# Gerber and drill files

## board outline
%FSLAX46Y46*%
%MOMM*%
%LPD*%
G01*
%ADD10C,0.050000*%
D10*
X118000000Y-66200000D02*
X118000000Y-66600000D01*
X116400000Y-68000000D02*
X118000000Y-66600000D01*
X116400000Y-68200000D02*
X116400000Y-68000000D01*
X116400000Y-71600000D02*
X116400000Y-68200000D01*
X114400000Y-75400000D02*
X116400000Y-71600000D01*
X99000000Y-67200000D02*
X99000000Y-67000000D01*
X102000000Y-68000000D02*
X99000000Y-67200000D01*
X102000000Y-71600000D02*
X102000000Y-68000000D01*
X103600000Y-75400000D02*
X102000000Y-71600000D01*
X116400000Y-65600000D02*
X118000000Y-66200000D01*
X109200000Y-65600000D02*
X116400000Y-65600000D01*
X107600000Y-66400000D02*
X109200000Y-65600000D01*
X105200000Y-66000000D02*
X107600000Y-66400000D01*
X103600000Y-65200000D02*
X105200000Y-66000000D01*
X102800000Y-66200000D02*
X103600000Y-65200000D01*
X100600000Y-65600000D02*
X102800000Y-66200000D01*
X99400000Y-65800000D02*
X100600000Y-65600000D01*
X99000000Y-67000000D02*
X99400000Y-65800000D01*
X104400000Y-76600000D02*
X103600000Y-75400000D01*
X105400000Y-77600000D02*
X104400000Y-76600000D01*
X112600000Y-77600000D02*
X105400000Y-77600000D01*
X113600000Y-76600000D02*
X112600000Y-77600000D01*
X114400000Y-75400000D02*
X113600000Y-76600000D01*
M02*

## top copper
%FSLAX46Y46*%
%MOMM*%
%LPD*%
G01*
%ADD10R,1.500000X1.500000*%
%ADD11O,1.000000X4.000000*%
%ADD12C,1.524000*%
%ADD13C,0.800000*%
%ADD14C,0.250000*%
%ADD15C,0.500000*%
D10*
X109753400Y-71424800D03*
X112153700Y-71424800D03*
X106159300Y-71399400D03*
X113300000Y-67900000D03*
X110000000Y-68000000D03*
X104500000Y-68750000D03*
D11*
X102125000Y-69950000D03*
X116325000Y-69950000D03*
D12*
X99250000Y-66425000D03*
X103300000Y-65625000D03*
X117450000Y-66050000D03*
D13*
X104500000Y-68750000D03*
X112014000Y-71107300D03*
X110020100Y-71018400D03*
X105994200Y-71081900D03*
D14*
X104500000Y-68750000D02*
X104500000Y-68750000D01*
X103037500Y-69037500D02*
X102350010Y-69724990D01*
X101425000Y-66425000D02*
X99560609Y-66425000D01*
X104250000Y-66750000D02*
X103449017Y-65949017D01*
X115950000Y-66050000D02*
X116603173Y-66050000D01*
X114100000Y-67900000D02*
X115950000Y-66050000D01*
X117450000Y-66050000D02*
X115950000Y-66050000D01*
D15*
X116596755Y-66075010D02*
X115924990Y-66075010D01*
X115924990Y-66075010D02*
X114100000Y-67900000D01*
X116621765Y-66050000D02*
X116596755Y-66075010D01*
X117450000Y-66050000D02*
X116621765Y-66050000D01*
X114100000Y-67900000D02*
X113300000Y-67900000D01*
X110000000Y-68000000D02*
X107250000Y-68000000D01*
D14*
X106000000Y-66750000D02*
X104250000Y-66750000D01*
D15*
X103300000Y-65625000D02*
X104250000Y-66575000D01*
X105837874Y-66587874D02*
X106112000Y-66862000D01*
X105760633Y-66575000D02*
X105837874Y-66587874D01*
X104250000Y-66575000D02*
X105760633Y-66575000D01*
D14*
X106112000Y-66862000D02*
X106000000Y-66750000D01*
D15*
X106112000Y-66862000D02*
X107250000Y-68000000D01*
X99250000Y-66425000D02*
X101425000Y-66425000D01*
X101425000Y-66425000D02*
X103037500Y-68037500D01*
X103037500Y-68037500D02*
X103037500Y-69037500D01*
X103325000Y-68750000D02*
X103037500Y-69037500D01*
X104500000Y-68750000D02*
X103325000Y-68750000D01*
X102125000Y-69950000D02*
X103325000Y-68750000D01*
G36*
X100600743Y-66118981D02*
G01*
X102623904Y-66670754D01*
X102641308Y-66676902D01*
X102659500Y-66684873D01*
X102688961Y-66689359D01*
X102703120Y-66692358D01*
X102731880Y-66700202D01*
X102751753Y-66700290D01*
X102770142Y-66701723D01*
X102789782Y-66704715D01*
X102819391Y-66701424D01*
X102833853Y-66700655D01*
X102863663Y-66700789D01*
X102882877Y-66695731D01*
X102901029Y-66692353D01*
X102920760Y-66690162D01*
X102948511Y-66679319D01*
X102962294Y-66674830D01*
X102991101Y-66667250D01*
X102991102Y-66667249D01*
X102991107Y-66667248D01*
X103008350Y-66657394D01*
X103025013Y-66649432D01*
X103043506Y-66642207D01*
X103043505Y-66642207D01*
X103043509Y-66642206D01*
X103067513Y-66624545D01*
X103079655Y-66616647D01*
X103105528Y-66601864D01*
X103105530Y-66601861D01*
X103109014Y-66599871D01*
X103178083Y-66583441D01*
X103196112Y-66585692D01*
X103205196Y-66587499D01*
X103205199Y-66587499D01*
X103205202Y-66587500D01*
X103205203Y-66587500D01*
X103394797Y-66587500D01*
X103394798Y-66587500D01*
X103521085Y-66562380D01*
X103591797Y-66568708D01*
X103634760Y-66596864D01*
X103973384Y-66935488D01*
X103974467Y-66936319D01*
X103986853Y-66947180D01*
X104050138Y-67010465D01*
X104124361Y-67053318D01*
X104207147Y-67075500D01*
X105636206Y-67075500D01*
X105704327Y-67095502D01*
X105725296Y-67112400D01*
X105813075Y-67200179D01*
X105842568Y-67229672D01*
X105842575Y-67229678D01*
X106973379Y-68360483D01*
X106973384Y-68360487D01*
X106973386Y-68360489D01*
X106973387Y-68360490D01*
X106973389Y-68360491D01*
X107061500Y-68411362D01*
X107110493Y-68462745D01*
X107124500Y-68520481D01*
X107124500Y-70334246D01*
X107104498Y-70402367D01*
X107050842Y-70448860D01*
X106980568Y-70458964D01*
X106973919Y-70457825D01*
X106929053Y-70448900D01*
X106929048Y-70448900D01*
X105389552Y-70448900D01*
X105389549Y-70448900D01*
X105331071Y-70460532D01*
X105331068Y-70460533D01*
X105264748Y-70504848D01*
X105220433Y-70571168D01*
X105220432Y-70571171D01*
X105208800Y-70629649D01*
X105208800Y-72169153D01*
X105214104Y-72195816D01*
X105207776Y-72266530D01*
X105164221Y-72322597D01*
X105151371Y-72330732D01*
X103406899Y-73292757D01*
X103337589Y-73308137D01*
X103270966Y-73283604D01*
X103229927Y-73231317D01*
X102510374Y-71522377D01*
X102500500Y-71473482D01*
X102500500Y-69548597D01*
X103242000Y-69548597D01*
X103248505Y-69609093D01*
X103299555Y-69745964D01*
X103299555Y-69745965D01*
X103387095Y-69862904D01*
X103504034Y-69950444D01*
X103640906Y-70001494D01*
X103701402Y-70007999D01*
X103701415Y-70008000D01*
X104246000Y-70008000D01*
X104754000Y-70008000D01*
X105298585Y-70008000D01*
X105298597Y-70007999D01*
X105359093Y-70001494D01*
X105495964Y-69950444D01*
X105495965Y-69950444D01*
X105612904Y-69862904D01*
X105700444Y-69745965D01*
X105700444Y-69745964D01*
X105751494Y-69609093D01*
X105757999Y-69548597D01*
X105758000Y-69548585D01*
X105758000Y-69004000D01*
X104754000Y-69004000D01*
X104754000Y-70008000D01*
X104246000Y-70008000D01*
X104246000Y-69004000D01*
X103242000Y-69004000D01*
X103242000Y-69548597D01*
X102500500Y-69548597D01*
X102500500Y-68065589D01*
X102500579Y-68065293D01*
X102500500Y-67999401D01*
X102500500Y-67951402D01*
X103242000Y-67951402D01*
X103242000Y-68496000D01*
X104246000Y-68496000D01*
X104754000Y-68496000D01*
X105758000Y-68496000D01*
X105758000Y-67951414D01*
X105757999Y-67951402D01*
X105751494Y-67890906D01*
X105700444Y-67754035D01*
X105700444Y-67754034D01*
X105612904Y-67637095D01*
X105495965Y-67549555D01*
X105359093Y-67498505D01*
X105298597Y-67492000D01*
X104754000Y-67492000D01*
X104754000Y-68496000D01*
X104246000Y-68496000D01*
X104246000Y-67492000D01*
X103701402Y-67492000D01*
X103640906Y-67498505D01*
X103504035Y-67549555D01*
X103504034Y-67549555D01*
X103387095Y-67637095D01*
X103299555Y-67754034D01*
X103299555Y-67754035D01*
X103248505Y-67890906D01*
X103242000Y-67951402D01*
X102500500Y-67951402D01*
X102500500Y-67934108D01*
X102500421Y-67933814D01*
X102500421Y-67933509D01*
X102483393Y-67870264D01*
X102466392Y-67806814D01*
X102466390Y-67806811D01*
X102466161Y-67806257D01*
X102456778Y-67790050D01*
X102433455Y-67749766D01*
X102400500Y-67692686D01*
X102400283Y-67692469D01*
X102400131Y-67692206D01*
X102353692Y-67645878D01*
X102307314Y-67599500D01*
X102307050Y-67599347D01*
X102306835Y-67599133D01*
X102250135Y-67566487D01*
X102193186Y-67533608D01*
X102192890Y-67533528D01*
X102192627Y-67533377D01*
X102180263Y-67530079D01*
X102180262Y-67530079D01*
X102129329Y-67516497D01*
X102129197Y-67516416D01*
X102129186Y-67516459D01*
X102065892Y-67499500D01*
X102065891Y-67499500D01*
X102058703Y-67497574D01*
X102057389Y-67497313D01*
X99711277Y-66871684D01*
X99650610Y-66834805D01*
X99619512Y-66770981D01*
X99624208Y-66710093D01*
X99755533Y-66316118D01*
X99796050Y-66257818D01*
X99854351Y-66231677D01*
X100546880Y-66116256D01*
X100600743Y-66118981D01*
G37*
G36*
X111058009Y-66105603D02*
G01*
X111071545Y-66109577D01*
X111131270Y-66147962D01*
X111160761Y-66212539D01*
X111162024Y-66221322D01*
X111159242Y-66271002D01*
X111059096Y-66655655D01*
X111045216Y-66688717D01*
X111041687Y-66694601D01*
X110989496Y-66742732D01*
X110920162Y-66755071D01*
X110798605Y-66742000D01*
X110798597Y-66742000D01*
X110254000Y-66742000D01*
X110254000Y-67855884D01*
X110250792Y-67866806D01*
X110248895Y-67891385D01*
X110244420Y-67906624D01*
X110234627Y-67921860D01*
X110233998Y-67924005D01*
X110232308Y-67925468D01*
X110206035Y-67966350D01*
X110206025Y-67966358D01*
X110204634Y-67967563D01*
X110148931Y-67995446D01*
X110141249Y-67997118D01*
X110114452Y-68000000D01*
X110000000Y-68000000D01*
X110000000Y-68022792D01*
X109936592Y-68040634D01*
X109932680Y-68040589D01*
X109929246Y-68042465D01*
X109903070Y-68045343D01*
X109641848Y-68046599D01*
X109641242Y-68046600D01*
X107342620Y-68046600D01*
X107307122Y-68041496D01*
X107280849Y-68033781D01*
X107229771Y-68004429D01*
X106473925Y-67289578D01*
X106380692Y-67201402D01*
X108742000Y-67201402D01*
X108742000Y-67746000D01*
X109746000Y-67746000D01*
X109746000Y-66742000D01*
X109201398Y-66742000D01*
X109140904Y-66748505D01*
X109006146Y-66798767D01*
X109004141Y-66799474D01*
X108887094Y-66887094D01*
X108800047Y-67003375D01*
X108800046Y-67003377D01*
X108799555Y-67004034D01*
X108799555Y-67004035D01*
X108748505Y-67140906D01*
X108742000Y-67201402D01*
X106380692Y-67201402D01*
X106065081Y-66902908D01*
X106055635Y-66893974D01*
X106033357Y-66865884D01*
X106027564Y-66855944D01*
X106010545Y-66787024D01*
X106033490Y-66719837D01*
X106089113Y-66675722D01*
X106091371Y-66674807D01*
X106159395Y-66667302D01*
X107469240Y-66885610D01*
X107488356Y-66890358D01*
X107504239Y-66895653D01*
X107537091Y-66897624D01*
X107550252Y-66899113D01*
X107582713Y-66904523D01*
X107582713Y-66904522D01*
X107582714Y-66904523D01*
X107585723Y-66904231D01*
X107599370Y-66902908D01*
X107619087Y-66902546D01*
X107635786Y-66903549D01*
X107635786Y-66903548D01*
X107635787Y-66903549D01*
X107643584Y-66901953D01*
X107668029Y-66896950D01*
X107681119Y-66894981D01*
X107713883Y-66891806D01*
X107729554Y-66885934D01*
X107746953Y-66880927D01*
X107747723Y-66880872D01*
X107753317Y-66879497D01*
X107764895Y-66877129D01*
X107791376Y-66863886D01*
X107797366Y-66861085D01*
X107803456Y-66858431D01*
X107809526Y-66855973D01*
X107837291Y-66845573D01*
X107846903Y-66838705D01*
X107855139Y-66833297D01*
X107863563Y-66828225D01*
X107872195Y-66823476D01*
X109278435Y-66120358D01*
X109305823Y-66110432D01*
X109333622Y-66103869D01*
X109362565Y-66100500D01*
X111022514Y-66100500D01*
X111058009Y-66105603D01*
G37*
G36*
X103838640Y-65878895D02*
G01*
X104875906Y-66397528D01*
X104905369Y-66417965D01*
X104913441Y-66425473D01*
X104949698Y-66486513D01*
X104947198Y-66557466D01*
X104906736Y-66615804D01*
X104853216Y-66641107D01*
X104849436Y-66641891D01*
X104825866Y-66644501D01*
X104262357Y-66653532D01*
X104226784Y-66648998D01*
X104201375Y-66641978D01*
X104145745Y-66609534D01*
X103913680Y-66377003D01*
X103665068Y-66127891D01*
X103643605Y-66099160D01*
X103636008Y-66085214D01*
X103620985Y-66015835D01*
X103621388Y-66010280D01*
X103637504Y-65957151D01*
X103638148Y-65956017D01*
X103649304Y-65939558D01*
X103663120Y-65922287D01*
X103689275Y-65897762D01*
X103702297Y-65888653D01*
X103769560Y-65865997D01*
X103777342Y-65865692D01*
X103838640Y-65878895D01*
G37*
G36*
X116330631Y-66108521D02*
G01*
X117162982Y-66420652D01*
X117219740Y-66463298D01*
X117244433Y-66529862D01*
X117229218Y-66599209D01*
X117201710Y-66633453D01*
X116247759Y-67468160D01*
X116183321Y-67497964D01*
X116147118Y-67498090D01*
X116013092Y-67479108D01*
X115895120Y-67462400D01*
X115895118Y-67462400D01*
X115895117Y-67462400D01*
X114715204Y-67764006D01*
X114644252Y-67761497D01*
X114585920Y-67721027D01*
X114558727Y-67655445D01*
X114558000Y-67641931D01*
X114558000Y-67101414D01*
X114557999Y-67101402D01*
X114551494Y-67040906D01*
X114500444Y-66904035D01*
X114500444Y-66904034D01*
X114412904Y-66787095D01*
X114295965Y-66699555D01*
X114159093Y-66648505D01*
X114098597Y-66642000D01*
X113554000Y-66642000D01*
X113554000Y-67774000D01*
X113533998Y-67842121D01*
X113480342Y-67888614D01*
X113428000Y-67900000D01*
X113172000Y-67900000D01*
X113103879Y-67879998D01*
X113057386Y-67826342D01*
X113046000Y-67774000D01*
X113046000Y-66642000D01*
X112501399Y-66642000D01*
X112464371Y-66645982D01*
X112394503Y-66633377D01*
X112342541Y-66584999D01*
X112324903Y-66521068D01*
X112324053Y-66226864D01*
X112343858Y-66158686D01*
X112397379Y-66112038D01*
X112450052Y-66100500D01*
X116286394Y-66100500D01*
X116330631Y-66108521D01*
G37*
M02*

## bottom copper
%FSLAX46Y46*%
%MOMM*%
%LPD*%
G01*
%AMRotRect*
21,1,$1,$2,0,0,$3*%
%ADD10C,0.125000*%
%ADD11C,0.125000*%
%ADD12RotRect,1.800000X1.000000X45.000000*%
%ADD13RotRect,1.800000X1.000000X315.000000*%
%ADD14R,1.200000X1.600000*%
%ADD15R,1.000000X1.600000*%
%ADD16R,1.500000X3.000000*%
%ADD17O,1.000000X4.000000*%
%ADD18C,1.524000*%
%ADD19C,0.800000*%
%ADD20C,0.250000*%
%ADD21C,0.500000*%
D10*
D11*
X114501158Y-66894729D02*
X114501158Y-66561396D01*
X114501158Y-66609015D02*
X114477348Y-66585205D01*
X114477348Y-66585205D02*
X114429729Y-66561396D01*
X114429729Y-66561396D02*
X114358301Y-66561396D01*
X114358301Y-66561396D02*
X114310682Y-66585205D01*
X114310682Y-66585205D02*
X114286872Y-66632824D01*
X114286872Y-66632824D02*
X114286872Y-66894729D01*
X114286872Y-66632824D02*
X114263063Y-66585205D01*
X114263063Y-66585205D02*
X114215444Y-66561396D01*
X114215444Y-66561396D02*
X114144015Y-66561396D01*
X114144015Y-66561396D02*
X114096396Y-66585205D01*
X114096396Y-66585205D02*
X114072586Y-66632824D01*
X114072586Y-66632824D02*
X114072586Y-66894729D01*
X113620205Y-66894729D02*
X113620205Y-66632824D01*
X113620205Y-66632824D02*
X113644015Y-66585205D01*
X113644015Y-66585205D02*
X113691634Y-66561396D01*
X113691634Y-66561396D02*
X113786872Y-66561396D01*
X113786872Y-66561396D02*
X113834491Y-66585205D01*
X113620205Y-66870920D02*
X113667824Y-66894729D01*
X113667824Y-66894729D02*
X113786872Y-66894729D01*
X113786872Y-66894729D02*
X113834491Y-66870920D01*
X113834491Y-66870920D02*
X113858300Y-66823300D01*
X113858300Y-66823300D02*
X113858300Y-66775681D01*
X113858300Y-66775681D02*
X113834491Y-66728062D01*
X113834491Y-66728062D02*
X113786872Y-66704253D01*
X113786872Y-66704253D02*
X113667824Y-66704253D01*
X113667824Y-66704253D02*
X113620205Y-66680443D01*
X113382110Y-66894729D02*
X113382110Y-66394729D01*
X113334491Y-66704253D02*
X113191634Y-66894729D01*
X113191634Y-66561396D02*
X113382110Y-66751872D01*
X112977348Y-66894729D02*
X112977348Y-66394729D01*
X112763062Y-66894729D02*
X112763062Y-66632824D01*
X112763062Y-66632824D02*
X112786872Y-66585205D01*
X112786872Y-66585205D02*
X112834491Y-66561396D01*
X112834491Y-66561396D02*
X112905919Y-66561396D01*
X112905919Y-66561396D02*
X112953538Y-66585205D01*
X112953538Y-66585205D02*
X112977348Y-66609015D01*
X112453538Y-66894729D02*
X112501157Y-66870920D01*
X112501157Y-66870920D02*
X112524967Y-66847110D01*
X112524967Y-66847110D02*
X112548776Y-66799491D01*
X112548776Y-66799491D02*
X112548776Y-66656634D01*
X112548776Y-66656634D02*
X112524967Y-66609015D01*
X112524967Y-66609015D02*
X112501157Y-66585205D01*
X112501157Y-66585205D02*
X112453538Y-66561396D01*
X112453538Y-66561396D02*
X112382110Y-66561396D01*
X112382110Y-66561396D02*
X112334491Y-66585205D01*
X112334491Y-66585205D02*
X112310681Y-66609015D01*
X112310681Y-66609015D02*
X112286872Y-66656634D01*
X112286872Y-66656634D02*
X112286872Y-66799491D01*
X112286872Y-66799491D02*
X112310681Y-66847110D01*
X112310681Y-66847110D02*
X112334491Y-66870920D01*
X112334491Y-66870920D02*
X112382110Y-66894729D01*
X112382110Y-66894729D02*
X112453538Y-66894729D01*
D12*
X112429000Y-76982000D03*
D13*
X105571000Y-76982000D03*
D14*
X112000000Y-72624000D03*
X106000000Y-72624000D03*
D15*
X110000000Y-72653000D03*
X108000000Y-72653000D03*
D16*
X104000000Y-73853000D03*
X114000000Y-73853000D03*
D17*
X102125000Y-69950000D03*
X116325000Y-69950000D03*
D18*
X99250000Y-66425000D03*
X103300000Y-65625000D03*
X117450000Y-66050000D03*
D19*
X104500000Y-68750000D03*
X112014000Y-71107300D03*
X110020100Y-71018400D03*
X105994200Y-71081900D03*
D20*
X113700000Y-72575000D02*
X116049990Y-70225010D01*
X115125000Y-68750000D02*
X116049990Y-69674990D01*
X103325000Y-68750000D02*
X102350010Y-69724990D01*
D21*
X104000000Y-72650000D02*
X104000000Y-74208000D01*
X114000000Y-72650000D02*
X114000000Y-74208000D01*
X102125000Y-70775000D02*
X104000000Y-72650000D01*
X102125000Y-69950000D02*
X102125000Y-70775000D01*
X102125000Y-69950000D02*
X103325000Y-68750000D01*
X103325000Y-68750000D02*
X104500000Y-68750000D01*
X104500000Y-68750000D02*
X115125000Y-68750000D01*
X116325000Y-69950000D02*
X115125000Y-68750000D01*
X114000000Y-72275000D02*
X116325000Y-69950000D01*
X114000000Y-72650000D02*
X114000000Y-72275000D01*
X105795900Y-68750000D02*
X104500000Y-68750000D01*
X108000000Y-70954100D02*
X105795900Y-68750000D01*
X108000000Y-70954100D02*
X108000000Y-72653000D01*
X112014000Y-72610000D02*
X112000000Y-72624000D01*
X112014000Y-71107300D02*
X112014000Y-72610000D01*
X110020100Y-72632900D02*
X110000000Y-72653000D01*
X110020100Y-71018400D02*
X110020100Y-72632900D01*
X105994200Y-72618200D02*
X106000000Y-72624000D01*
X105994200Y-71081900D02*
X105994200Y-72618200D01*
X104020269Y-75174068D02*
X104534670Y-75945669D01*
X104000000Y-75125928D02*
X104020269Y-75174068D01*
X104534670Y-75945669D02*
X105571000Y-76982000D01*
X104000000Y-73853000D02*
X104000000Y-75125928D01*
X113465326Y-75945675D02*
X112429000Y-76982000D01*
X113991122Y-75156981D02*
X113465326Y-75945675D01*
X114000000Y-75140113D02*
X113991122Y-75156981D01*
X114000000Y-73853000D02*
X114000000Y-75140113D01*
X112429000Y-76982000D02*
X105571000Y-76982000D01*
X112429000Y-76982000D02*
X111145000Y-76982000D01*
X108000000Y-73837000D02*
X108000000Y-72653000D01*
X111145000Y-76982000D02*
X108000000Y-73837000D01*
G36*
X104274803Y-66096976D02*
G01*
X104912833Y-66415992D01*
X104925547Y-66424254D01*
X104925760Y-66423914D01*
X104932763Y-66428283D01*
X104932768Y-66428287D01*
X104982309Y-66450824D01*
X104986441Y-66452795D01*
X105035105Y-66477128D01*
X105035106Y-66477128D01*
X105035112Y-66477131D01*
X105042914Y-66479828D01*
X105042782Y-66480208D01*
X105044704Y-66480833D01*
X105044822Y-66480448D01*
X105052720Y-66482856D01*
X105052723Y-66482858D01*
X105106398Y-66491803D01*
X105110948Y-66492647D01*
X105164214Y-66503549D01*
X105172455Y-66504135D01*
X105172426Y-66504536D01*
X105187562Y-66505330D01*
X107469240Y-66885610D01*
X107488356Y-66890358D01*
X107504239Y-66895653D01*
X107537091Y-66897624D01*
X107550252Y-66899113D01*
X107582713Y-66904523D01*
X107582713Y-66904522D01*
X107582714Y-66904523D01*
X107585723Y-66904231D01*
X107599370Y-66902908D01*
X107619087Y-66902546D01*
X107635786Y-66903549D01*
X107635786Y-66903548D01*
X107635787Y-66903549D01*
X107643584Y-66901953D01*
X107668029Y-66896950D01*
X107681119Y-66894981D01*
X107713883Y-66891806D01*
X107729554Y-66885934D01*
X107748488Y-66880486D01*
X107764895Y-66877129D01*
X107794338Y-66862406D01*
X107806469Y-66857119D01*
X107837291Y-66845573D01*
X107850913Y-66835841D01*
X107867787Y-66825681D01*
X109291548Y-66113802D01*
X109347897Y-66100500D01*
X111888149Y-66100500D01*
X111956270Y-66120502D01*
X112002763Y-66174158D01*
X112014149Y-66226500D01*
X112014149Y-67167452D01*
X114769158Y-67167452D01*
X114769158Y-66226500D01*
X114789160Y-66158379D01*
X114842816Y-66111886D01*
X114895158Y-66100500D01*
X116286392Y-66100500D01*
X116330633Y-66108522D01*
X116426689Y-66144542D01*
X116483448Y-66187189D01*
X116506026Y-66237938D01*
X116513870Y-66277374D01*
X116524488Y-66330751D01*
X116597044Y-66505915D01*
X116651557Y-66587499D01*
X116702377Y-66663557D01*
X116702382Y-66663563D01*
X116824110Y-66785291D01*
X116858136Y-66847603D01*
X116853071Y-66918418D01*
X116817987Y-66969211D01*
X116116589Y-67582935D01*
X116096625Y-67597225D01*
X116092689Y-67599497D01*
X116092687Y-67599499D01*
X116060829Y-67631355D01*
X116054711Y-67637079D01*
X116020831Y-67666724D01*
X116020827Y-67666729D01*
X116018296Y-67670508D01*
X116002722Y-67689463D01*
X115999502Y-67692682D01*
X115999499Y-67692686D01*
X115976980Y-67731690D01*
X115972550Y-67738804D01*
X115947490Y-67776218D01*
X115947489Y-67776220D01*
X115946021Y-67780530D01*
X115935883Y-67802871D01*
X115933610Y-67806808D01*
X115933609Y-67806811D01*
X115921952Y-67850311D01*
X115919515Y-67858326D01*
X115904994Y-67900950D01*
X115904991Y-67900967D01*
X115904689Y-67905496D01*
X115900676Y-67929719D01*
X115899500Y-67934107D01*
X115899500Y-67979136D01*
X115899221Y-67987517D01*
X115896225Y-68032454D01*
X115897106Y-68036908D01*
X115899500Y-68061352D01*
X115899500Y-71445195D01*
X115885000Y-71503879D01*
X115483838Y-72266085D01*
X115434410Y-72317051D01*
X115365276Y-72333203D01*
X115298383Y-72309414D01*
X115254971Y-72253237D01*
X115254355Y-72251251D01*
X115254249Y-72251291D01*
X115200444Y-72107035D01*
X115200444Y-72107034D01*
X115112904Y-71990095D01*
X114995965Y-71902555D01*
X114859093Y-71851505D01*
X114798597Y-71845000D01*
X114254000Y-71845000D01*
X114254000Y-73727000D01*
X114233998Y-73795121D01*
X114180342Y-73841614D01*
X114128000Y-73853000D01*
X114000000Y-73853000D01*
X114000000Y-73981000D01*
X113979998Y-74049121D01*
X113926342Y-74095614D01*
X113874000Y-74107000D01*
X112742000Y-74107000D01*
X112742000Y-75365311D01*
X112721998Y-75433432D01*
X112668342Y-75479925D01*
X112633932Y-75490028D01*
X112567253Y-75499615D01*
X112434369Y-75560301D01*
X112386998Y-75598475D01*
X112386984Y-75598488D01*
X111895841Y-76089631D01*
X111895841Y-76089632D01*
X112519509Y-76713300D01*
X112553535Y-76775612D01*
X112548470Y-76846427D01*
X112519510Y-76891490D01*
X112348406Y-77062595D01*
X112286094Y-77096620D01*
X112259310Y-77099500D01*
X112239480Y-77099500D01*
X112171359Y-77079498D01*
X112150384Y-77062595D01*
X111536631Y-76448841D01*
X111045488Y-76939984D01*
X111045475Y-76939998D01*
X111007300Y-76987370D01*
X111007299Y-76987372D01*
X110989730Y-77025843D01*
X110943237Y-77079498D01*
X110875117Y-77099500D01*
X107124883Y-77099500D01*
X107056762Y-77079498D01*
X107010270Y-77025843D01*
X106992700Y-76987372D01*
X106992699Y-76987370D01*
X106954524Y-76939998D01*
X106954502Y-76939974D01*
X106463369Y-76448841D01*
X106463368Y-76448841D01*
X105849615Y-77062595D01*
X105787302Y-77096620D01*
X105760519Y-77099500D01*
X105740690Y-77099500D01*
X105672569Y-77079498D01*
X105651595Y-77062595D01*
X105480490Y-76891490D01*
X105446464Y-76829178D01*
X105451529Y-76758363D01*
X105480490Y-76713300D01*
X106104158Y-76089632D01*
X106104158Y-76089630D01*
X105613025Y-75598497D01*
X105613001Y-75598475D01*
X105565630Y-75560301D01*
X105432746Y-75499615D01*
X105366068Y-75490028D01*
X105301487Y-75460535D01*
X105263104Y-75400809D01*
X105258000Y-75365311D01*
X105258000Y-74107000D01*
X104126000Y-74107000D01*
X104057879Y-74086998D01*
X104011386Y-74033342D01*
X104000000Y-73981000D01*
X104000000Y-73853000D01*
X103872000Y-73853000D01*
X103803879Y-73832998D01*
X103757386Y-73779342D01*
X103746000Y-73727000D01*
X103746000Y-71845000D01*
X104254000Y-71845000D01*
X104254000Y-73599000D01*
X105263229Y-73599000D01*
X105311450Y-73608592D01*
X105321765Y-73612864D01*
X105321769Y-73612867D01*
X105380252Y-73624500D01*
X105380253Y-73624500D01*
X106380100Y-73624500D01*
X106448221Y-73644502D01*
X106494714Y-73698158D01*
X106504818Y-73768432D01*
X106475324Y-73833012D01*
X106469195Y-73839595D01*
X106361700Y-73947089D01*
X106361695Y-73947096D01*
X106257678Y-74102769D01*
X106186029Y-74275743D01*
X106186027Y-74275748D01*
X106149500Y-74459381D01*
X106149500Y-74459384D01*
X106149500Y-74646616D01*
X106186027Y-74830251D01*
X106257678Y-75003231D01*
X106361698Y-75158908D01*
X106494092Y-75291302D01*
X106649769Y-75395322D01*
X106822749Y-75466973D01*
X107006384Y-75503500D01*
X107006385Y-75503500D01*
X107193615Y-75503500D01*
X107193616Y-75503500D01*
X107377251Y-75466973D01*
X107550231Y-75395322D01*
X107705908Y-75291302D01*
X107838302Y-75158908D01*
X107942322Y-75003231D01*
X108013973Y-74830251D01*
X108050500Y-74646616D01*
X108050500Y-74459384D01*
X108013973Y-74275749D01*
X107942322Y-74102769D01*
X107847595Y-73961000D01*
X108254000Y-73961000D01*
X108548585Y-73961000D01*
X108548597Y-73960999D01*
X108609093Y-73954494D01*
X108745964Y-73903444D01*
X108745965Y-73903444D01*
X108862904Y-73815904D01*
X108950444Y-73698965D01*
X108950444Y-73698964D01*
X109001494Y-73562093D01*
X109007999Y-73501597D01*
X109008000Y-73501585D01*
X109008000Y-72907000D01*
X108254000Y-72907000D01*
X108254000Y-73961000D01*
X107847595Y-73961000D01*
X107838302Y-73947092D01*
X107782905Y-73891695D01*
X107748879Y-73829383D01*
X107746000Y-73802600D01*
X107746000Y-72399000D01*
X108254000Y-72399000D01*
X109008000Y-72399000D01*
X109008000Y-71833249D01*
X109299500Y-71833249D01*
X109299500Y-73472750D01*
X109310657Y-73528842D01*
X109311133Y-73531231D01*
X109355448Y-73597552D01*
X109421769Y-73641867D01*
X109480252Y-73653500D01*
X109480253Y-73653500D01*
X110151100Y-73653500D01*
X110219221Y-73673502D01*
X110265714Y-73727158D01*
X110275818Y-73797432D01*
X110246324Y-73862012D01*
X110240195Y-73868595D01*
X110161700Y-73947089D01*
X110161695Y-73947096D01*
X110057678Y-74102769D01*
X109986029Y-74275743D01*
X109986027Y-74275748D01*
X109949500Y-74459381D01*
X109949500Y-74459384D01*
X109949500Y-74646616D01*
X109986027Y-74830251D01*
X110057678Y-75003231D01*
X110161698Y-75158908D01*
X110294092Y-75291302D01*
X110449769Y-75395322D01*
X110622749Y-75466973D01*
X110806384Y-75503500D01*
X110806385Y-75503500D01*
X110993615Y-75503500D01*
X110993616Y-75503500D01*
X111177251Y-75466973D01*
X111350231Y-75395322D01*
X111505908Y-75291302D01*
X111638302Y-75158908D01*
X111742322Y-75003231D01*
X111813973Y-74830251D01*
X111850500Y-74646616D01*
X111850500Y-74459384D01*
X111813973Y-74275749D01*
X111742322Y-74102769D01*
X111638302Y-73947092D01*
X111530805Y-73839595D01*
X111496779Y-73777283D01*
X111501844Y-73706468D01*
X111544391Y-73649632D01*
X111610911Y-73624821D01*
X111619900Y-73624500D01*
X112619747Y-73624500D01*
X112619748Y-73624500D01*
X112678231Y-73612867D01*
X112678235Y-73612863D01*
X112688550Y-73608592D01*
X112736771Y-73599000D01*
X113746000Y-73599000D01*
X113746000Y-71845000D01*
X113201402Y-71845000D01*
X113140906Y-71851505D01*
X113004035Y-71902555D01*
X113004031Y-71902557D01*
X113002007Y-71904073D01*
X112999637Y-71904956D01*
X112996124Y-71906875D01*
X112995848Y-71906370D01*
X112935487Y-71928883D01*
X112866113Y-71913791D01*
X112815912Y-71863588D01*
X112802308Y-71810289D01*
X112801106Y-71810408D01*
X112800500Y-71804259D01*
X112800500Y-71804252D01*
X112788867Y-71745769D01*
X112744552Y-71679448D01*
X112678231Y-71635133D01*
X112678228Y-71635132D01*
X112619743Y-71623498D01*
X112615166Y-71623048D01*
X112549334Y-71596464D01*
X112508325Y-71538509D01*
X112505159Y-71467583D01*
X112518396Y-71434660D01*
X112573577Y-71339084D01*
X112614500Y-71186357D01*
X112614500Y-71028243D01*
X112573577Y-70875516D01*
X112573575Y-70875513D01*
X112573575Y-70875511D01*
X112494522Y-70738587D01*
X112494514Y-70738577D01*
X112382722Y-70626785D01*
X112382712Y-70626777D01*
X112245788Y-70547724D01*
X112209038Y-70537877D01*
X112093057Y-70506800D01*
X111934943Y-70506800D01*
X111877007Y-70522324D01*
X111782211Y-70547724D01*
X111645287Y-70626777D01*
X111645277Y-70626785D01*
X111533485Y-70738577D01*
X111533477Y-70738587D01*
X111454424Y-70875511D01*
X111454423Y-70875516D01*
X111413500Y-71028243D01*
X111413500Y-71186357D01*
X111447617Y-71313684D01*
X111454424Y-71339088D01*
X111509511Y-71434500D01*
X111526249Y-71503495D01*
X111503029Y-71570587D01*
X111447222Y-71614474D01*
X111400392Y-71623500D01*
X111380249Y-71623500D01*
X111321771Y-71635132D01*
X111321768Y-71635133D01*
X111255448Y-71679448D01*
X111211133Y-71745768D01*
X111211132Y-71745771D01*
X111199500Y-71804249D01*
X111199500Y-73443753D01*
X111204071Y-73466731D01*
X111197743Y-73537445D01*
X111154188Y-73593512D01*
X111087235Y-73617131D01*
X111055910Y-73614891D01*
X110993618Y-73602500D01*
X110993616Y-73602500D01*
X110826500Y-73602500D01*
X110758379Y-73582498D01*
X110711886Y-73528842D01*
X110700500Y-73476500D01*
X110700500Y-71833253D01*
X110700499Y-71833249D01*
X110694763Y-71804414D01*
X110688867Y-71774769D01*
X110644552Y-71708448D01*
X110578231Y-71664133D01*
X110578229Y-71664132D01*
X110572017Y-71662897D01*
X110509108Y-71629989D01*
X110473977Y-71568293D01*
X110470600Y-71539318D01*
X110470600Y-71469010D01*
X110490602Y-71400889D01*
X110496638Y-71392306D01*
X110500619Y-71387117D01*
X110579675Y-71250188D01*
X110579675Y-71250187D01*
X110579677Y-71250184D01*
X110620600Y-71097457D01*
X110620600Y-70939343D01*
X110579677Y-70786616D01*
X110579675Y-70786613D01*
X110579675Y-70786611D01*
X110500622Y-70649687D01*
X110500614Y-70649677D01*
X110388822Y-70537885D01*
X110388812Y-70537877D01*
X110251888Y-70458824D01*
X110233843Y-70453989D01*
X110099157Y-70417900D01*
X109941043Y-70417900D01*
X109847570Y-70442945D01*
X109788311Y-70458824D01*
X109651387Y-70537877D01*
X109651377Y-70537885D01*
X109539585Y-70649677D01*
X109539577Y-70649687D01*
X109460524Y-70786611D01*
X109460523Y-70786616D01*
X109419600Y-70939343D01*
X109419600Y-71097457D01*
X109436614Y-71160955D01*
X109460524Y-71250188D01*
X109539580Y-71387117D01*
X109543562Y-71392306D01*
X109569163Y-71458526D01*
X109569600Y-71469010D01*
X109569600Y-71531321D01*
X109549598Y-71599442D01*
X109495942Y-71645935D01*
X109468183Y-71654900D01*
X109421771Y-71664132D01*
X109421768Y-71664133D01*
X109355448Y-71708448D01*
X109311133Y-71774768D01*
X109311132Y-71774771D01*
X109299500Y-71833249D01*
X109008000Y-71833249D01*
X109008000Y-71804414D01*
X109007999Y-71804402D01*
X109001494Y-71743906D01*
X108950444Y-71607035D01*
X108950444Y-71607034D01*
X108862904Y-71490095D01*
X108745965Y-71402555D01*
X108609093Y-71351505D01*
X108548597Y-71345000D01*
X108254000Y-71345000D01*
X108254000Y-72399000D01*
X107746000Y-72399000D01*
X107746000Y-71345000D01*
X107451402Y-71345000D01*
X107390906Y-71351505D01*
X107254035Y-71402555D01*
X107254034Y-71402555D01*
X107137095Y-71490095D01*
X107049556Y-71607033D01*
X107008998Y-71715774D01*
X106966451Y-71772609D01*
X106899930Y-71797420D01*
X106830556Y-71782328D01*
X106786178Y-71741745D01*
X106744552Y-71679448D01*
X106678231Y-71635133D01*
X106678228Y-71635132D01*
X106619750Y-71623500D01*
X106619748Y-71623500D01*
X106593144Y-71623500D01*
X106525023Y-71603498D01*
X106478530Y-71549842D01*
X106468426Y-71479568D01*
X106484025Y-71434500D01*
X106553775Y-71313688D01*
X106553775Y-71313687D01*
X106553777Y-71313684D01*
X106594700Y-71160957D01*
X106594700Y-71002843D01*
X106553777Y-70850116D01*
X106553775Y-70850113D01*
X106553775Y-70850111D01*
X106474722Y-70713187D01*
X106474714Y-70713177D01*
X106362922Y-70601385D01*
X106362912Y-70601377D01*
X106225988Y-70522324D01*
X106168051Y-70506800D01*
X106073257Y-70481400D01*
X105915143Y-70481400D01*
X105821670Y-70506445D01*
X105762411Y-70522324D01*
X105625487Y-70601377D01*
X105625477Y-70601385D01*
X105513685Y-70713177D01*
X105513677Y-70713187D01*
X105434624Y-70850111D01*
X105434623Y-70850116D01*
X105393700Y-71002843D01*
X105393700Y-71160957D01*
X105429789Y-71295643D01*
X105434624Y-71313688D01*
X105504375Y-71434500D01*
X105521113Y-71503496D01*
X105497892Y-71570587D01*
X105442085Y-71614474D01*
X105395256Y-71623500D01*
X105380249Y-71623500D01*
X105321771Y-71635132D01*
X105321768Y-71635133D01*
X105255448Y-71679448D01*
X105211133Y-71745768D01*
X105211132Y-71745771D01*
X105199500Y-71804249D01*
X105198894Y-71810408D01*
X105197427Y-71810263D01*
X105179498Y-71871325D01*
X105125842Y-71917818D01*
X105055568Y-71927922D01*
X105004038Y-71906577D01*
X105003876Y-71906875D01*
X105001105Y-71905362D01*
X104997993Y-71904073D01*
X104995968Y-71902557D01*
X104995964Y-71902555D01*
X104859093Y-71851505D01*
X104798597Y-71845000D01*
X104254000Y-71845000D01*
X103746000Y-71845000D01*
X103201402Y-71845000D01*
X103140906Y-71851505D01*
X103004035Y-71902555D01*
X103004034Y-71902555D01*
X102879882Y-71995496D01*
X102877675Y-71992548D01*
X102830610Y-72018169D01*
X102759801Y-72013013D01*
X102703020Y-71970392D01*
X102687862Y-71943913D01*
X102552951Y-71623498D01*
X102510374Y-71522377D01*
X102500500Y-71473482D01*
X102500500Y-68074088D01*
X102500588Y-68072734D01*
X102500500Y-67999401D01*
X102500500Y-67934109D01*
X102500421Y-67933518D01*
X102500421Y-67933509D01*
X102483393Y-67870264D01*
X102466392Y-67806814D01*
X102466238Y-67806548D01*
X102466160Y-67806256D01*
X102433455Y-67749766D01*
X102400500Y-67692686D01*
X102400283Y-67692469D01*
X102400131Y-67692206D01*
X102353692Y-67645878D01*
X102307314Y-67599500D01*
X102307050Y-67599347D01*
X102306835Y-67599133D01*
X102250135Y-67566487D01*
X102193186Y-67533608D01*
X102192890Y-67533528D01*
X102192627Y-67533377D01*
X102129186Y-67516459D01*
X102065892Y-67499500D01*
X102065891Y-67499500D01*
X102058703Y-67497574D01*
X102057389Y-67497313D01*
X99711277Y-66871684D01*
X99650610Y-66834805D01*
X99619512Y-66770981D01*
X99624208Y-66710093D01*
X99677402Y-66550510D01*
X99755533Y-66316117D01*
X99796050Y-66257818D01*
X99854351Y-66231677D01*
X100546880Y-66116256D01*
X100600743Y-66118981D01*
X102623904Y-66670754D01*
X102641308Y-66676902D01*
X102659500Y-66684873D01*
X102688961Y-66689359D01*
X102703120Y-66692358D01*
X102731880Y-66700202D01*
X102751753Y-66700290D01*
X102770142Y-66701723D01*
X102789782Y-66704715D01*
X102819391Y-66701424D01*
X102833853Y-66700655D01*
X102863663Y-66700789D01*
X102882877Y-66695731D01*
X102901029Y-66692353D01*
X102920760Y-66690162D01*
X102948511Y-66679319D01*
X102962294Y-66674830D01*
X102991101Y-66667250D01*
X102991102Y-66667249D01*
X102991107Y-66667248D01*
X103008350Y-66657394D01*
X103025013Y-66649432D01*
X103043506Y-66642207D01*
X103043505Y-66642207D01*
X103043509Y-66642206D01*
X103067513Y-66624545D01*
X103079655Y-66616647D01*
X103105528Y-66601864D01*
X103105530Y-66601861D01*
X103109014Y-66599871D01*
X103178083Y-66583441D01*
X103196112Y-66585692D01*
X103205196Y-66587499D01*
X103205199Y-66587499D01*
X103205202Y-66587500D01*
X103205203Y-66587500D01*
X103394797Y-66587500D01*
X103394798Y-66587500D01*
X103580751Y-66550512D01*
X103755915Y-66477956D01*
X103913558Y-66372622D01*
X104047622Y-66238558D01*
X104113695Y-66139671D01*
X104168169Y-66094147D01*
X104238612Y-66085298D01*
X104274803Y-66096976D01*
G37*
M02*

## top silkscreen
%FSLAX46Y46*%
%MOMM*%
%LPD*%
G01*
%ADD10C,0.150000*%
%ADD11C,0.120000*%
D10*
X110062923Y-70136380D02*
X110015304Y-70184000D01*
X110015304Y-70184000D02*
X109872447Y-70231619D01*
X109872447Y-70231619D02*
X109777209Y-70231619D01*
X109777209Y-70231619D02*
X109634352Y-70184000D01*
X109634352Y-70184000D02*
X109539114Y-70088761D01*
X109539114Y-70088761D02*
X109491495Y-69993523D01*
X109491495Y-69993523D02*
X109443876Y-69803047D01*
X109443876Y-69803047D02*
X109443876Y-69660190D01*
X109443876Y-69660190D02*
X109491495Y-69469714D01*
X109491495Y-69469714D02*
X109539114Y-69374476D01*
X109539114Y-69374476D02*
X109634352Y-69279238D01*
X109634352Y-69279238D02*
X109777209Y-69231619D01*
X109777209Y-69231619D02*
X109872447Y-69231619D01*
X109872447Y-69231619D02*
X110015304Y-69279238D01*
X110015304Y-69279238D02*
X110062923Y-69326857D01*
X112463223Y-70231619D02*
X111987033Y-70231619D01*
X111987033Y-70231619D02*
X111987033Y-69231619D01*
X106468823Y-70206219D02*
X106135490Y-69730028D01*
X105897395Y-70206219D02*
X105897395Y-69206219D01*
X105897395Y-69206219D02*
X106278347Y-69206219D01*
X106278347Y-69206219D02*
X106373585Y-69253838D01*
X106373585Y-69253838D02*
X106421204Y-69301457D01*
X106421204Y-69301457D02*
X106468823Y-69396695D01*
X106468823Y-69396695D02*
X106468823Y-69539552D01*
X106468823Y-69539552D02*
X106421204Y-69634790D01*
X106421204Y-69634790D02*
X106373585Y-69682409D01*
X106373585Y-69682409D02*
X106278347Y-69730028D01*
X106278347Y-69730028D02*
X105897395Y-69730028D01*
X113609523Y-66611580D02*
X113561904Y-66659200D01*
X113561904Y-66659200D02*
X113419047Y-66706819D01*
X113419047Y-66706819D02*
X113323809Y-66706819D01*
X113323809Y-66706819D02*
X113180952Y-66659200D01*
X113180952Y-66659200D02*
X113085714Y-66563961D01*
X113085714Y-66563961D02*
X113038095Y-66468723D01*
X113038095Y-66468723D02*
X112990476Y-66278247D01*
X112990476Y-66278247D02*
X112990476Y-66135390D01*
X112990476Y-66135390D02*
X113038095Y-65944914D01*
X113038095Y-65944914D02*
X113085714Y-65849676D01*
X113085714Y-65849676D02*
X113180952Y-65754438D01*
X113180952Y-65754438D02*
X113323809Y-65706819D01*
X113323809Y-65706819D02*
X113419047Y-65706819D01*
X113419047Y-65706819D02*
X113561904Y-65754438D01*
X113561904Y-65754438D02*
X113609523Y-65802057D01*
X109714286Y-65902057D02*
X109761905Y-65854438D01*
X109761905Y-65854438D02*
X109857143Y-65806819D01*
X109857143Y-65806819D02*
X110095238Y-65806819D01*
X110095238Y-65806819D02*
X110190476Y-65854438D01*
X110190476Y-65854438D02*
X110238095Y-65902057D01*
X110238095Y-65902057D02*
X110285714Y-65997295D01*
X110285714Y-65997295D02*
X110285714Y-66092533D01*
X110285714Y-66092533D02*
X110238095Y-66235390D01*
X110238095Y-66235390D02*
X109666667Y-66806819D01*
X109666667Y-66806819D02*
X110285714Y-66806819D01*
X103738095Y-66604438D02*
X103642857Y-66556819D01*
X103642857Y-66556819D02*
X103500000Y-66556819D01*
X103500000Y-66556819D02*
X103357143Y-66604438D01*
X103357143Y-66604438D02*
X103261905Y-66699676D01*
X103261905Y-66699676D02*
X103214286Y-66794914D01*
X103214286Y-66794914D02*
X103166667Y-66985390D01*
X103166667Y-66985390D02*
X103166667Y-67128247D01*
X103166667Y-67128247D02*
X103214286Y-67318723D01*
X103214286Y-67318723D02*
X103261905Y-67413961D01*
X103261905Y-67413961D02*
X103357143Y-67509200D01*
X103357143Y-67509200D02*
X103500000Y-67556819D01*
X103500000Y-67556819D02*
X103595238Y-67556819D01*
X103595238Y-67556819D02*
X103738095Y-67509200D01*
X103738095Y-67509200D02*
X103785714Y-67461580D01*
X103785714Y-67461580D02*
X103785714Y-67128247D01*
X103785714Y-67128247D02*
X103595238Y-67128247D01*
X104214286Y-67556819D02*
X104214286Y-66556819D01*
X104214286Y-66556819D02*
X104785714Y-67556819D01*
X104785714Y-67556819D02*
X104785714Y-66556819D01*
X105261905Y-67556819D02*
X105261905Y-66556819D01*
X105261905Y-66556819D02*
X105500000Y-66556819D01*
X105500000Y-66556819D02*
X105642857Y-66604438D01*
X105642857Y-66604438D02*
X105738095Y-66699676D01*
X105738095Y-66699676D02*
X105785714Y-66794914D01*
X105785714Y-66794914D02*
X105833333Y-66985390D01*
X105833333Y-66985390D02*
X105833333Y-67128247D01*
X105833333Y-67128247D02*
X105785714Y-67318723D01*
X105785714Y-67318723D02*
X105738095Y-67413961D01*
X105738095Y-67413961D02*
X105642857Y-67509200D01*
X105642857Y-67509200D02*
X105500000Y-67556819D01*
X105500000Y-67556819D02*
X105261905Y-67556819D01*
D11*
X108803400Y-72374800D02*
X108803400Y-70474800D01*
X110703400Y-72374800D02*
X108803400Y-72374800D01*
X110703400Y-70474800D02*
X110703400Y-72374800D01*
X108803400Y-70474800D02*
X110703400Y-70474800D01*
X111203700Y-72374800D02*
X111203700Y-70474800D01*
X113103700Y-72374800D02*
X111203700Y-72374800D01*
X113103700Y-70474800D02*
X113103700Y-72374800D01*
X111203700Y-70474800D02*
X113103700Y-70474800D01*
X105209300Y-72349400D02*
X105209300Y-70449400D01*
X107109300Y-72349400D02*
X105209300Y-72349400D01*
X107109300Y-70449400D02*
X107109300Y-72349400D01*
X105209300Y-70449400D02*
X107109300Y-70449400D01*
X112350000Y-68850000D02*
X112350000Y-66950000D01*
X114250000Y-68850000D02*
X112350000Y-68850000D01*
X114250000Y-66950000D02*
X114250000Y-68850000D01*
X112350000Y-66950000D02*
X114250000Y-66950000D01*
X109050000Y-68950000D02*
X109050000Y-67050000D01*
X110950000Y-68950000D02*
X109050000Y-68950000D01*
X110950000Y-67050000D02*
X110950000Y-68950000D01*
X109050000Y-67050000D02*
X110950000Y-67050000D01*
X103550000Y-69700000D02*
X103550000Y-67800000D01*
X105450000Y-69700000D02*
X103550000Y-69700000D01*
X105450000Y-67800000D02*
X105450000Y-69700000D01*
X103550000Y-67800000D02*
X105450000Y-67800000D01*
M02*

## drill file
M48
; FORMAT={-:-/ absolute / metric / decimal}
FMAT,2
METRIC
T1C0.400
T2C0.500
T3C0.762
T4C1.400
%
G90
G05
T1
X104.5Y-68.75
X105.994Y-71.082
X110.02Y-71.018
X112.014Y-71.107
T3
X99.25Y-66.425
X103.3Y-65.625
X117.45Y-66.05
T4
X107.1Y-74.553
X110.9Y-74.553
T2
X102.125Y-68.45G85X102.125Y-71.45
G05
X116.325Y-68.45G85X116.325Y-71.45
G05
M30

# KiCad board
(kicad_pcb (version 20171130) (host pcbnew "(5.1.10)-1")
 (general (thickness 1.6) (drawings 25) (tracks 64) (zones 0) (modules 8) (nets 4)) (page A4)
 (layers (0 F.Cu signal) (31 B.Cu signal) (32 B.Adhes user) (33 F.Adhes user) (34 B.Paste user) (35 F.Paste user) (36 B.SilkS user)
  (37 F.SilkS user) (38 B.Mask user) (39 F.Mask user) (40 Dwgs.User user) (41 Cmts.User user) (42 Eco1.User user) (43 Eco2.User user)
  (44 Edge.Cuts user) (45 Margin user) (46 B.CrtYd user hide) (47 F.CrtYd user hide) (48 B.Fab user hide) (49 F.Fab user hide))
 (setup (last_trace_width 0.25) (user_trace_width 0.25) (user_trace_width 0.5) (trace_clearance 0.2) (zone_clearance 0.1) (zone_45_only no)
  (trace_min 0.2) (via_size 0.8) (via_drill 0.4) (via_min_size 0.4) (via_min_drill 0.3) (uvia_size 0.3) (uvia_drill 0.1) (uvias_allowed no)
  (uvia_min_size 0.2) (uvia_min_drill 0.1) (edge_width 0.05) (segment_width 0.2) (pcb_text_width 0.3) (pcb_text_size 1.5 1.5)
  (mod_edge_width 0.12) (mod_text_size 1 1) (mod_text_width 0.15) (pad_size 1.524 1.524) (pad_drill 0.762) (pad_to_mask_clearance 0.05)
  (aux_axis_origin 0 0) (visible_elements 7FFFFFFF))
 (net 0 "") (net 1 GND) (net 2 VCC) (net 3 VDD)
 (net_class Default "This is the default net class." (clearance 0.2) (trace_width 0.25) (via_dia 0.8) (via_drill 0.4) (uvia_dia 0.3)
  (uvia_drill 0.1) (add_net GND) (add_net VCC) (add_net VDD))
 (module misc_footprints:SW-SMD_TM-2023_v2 (layer B.Cu) (at 109 74.803)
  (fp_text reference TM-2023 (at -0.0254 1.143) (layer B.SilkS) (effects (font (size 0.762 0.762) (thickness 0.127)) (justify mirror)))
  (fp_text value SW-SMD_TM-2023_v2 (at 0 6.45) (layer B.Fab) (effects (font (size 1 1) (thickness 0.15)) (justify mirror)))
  (pad GND smd rect (at 3.429 2.179 45) (size 1.8 1) (layers B.Cu B.Paste B.Mask) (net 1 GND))
  (pad GND smd rect (at -3.429 2.179 315) (size 1.8 1) (layers B.Cu B.Paste B.Mask) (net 1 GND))
  (pad 1 smd rect (at 3 -2.179) (size 1.2 1.6) (layers B.Cu B.Paste B.Mask))
  (pad 2 smd rect (at -3 -2.179) (size 1.2 1.6) (layers B.Cu B.Paste B.Mask))
  (pad C smd rect (at 1 -2.15) (size 1 1.6) (layers B.Cu B.Paste B.Mask))
  (pad T smd rect (at -1 -2.15) (size 1 1.6) (layers B.Cu B.Paste B.Mask) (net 1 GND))
  (pad GND smd rect (at -5 -0.95) (size 1.5 3) (layers B.Cu B.Paste B.Mask) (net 1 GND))
  (pad 6 smd rect (at 5 -0.95) (size 1.5 3) (layers B.Cu B.Paste B.Mask) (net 1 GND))
  (pad "" np_thru_hole circle (at 1.9 -0.25) (size 1.4 1.4) (drill 1.4) (layers *.Cu *.Mask))
  (pad "" np_thru_hole circle (at -1.9 -0.25) (size 1.4 1.4) (drill 1.4) (layers *.Cu *.Mask)))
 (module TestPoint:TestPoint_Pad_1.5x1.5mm (layer F.Cu) (at 109.7534 71.4248)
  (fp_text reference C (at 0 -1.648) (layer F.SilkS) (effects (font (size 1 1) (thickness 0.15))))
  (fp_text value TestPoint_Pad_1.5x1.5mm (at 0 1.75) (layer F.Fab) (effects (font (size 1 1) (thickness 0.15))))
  (fp_line (start -0.95 0.95) (end -0.95 -0.95) (layer F.SilkS) (width 0.12))
  (fp_line (start 0.95 0.95) (end -0.95 0.95) (layer F.SilkS) (width 0.12))
  (fp_line (start 0.95 -0.95) (end 0.95 0.95) (layer F.SilkS) (width 0.12))
  (fp_line (start -0.95 -0.95) (end 0.95 -0.95) (layer F.SilkS) (width 0.12))
  (pad 1 smd rect (at 0 0) (size 1.5 1.5) (layers F.Cu F.Mask)))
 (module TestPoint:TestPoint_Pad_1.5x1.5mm (layer F.Cu) (at 112.1537 71.4248)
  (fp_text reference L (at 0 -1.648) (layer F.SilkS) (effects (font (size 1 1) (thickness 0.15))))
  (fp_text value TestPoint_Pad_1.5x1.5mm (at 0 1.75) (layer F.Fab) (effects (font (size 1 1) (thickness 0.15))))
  (fp_line (start -0.95 0.95) (end -0.95 -0.95) (layer F.SilkS) (width 0.12))
  (fp_line (start 0.95 0.95) (end -0.95 0.95) (layer F.SilkS) (width 0.12))
  (fp_line (start 0.95 -0.95) (end 0.95 0.95) (layer F.SilkS) (width 0.12))
  (fp_line (start -0.95 -0.95) (end 0.95 -0.95) (layer F.SilkS) (width 0.12))
  (pad 1 smd rect (at 0 0) (size 1.5 1.5) (layers F.Cu F.Mask)))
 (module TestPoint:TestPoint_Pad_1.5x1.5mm (layer F.Cu) (at 106.1593 71.3994)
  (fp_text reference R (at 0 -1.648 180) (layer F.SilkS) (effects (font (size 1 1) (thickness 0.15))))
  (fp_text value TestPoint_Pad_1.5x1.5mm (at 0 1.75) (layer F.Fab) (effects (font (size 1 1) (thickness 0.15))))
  (fp_line (start -0.95 0.95) (end -0.95 -0.95) (layer F.SilkS) (width 0.12))
  (fp_line (start 0.95 0.95) (end -0.95 0.95) (layer F.SilkS) (width 0.12))
  (fp_line (start 0.95 -0.95) (end 0.95 0.95) (layer F.SilkS) (width 0.12))
  (fp_line (start -0.95 -0.95) (end 0.95 -0.95) (layer F.SilkS) (width 0.12))
  (pad 1 smd rect (at 0 0) (size 1.5 1.5) (layers F.Cu F.Mask)))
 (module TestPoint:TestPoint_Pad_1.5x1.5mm (layer F.Cu) (at 113.3 67.9)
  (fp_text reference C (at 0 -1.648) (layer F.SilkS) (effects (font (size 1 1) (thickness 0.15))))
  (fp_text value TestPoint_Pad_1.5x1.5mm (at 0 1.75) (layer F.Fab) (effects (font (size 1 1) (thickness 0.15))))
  (fp_line (start -0.95 0.95) (end -0.95 -0.95) (layer F.SilkS) (width 0.12))
  (fp_line (start 0.95 0.95) (end -0.95 0.95) (layer F.SilkS) (width 0.12))
  (fp_line (start 0.95 -0.95) (end 0.95 0.95) (layer F.SilkS) (width 0.12))
  (fp_line (start -0.95 -0.95) (end 0.95 -0.95) (layer F.SilkS) (width 0.12))
  (pad 1 smd rect (at 0 0) (size 1.5 1.5) (layers F.Cu F.Mask) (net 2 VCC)))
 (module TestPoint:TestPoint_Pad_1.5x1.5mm (layer F.Cu) (at 110 68)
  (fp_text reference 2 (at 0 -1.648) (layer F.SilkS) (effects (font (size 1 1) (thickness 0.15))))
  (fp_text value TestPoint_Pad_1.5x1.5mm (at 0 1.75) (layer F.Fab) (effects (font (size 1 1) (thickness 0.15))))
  (fp_line (start -0.95 0.95) (end -0.95 -0.95) (layer F.SilkS) (width 0.12))
  (fp_line (start 0.95 0.95) (end -0.95 0.95) (layer F.SilkS) (width 0.12))
  (fp_line (start 0.95 -0.95) (end 0.95 0.95) (layer F.SilkS) (width 0.12))
  (fp_line (start -0.95 -0.95) (end 0.95 -0.95) (layer F.SilkS) (width 0.12))
  (pad 1 smd rect (at 0 0) (size 1.5 1.5) (layers F.Cu F.Mask) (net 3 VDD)))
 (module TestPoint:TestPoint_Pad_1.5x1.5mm (layer F.Cu) (at 104.5 68.75)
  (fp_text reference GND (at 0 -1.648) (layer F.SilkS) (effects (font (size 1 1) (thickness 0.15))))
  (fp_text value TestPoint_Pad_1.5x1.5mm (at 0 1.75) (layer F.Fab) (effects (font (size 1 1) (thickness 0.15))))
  (fp_line (start -0.95 0.95) (end -0.95 -0.95) (layer F.SilkS) (width 0.12))
  (fp_line (start 0.95 0.95) (end -0.95 0.95) (layer F.SilkS) (width 0.12))
  (fp_line (start 0.95 -0.95) (end 0.95 0.95) (layer F.SilkS) (width 0.12))
  (fp_line (start -0.95 -0.95) (end 0.95 -0.95) (layer F.SilkS) (width 0.12))
  (pad 1 smd rect (at 0 0) (size 1.5 1.5) (layers F.Cu F.Mask) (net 1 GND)))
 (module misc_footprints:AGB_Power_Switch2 (layer F.Cu) (at 108.4 70.2)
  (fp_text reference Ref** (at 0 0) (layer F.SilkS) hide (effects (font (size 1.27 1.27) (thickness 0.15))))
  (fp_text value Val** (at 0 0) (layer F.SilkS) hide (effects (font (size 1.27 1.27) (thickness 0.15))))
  (pad 3 thru_hole oval (at -6.275 -0.25) (size 1 4) (drill oval 0.5 3.5) (layers *.Cu *.Mask) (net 1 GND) (zone_connect 2))
  (pad 3 thru_hole oval (at 7.925 -0.25) (size 1 4) (drill oval 0.5 3.5) (layers *.Cu *.Mask) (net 1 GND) (zone_connect 2))
  (pad 3 thru_hole circle (at -9.15 -3.775) (size 1.524 1.524) (drill 0.762) (layers *.Cu *.Mask) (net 1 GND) (zone_connect 2))
  (pad 2 thru_hole circle (at -5.1 -4.575) (size 1.524 1.524) (drill 0.762) (layers *.Cu *.Mask) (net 3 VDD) (zone_connect 2))
  (pad 1 thru_hole circle (at 9.05 -4.15) (size 1.524 1.524) (drill 0.762) (layers *.Cu *.Mask) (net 2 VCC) (zone_connect 2)))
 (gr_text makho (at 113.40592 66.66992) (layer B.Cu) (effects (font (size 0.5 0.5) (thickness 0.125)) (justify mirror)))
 (gr_line (start 118 66.2) (end 118 66.6) (layer Edge.Cuts) (width 0.05))
 (gr_line (start 116.4 68) (end 118 66.6) (layer Edge.Cuts) (width 0.05))
 (gr_line (start 116.4 68.2) (end 116.4 68) (layer Edge.Cuts) (width 0.05))
 (gr_line (start 116.4 71.6) (end 116.4 68.2) (layer Edge.Cuts) (width 0.05))
 (gr_line (start 114.4 75.4) (end 116.4 71.6) (layer Edge.Cuts) (width 0.05))
 (gr_line (start 99 67.2) (end 99 67) (layer Edge.Cuts) (width 0.05))
 (gr_line (start 102 68) (end 99 67.2) (layer Edge.Cuts) (width 0.05))
 (gr_line (start 102 71.6) (end 102 68) (layer Edge.Cuts) (width 0.05))
 (gr_line (start 103.6 75.4) (end 102 71.6) (layer Edge.Cuts) (width 0.05))
 (gr_line (start 116.4 65.6) (end 118 66.2) (layer Edge.Cuts) (width 0.05))
 (gr_line (start 109.2 65.6) (end 116.4 65.6) (layer Edge.Cuts) (width 0.05))
 (gr_line (start 107.6 66.4) (end 109.2 65.6) (layer Edge.Cuts) (width 0.05))
 (gr_line (start 105.2 66) (end 107.6 66.4) (layer Edge.Cuts) (width 0.05))
 (gr_line (start 103.6 65.2) (end 105.2 66) (layer Edge.Cuts) (width 0.05))
 (gr_line (start 102.8 66.2) (end 103.6 65.2) (layer Edge.Cuts) (width 0.05))
 (gr_line (start 100.6 65.6) (end 102.8 66.2) (layer Edge.Cuts) (width 0.05))
 (gr_line (start 99.4 65.8) (end 100.6 65.6) (layer Edge.Cuts) (width 0.05))
 (gr_line (start 99 67) (end 99.4 65.8) (layer Edge.Cuts) (width 0.05))
 (gr_line (start 104.4 76.6) (end 103.6 75.4) (layer Edge.Cuts) (width 0.05))
 (gr_line (start 105.4 77.6) (end 104.4 76.6) (layer Edge.Cuts) (width 0.05))
 (gr_line (start 112.6 77.6) (end 105.4 77.6) (layer Edge.Cuts) (width 0.05))
 (gr_line (start 113.6 76.6) (end 112.6 77.6) (layer Edge.Cuts) (width 0.05))
 (gr_line (start 114.4 75.4) (end 113.6 76.6) (layer Edge.Cuts) (width 0.05))
 (segment (start 113.7 72.575) (end 116.04999 70.22501) (width 0.25) (layer B.Cu) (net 1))
 (segment (start 104.5 68.75) (end 104.5 68.75) (width 0.25) (layer F.Cu) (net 1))
 (segment (start 103.0375 69.0375) (end 102.35001 69.72499) (width 0.25) (layer F.Cu) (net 1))
 (segment (start 101.425 66.425) (end 99.560609 66.425) (width 0.25) (layer F.Cu) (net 1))
 (segment (start 104.25 66.75) (end 103.449017 65.949017) (width 0.25) (layer F.Cu) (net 3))
 (segment (start 115.95 66.05) (end 116.603173 66.05) (width 0.25) (layer F.Cu) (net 2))
 (segment (start 114.1 67.9) (end 115.95 66.05) (width 0.25) (layer F.Cu) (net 2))
 (segment (start 117.45 66.05) (end 115.95 66.05) (width 0.25) (layer F.Cu) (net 2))
 (via (at 104.5 68.75) (size 0.8) (drill 0.4) (layers F.Cu B.Cu) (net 1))
 (segment (start 115.125 68.75) (end 116.04999 69.67499) (width 0.25) (layer B.Cu) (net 1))
 (segment (start 103.325 68.75) (end 102.35001 69.72499) (width 0.25) (layer B.Cu) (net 1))
 (segment (start 104 72.65) (end 104 74.208) (width 0.5) (layer B.Cu) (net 1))
 (segment (start 114 72.65) (end 114 74.208) (width 0.5) (layer B.Cu) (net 1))
 (segment (start 116.596755 66.07501) (end 115.92499 66.07501) (width 0.5) (layer F.Cu) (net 2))
 (segment (start 115.92499 66.07501) (end 114.1 67.9) (width 0.5) (layer F.Cu) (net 2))
 (segment (start 116.621765 66.05) (end 116.596755 66.07501) (width 0.5) (layer F.Cu) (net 2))
 (segment (start 117.45 66.05) (end 116.621765 66.05) (width 0.5) (layer F.Cu) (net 2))
 (segment (start 114.1 67.9) (end 113.3 67.9) (width 0.5) (layer F.Cu) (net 2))
 (segment (start 110 68) (end 107.25 68) (width 0.5) (layer F.Cu) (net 3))
 (segment (start 106 66.75) (end 104.25 66.75) (width 0.25) (layer F.Cu) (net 3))
 (segment (start 103.3 65.625) (end 104.25 66.575) (width 0.5) (layer F.Cu) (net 3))
 (segment (start 105.837874 66.587874) (end 106.112 66.862) (width 0.5) (layer F.Cu) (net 3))
 (segment (start 105.760633 66.575) (end 105.837874 66.587874) (width 0.5) (layer F.Cu) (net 3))
 (segment (start 104.25 66.575) (end 105.760633 66.575) (width 0.5) (layer F.Cu) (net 3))
 (segment (start 106.112 66.862) (end 106 66.75) (width 0.25) (layer F.Cu) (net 3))
 (segment (start 106.112 66.862) (end 107.25 68) (width 0.5) (layer F.Cu) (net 3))
 (segment (start 99.25 66.425) (end 101.425 66.425) (width 0.5) (layer F.Cu) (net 1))
 (segment (start 101.425 66.425) (end 103.0375 68.0375) (width 0.5) (layer F.Cu) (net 1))
 (segment (start 103.0375 68.0375) (end 103.0375 69.0375) (width 0.5) (layer F.Cu) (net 1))
 (segment (start 103.325 68.75) (end 103.0375 69.0375) (width 0.5) (layer F.Cu) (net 1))
 (segment (start 104.5 68.75) (end 103.325 68.75) (width 0.5) (layer F.Cu) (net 1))
 (segment (start 102.125 69.95) (end 103.325 68.75) (width 0.5) (layer F.Cu) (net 1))
 (segment (start 102.125 70.775) (end 104 72.65) (width 0.5) (layer B.Cu) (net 1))
 (segment (start 102.125 69.95) (end 102.125 70.775) (width 0.5) (layer B.Cu) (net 1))
 (segment (start 102.125 69.95) (end 103.325 68.75) (width 0.5) (layer B.Cu) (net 1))
 (segment (start 103.325 68.75) (end 104.5 68.75) (width 0.5) (layer B.Cu) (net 1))
 (segment (start 104.5 68.75) (end 115.125 68.75) (width 0.5) (layer B.Cu) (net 1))
 (segment (start 116.325 69.95) (end 115.125 68.75) (width 0.5) (layer B.Cu) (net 1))
 (segment (start 114 72.275) (end 116.325 69.95) (width 0.5) (layer B.Cu) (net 1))
 (segment (start 114 72.65) (end 114 72.275) (width 0.5) (layer B.Cu) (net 1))
 (segment (start 105.7959 68.75) (end 104.5 68.75) (width 0.5) (layer B.Cu) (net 1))
 (segment (start 108 70.9541) (end 105.7959 68.75) (width 0.5) (layer B.Cu) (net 1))
 (via (at 112.014 71.1073) (size 0.8) (drill 0.4) (layers F.Cu B.Cu) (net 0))
 (via (at 110.0201 71.0184) (size 0.8) (drill 0.4) (layers F.Cu B.Cu) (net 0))
 (via (at 105.9942 71.0819) (size 0.8) (drill 0.4) (layers F.Cu B.Cu) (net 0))
 (segment (start 108 70.9541) (end 108 72.653) (width 0.5) (layer B.Cu) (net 1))
 (segment (start 112.014 72.61) (end 112 72.624) (width 0.5) (layer B.Cu) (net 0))
 (segment (start 112.014 71.1073) (end 112.014 72.61) (width 0.5) (layer B.Cu) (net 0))
 (segment (start 110.0201 72.6329) (end 110 72.653) (width 0.5) (layer B.Cu) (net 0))
 (segment (start 110.0201 71.0184) (end 110.0201 72.6329) (width 0.5) (layer B.Cu) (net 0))
 (segment (start 105.9942 72.6182) (end 106 72.624) (width 0.5) (layer B.Cu) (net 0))
 (segment (start 105.9942 71.0819) (end 105.9942 72.6182) (width 0.5) (layer B.Cu) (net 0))
 (segment (start 104.020269 75.174068) (end 104.53467 75.945669) (width 0.5) (layer B.Cu) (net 1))
 (segment (start 104 75.125928) (end 104.020269 75.174068) (width 0.5) (layer B.Cu) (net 1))
 (segment (start 104.53467 75.945669) (end 105.571 76.982) (width 0.5) (layer B.Cu) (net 1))
 (segment (start 104 73.853) (end 104 75.125928) (width 0.5) (layer B.Cu) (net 1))
 (segment (start 113.465326 75.945675) (end 112.429 76.982) (width 0.5) (layer B.Cu) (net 1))
 (segment (start 113.991122 75.156981) (end 113.465326 75.945675) (width 0.5) (layer B.Cu) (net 1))
 (segment (start 114 75.140113) (end 113.991122 75.156981) (width 0.5) (layer B.Cu) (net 1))
 (segment (start 114 73.853) (end 114 75.140113) (width 0.5) (layer B.Cu) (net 1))
 (segment (start 112.429 76.982) (end 105.571 76.982) (width 0.5) (layer B.Cu) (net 1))
 (segment (start 112.429 76.982) (end 111.145 76.982) (width 0.5) (layer B.Cu) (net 1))
 (segment (start 108 73.837) (end 108 72.653) (width 0.5) (layer B.Cu) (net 1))
 (segment (start 111.145 76.982) (end 108 73.837) (width 0.5) (layer B.Cu) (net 1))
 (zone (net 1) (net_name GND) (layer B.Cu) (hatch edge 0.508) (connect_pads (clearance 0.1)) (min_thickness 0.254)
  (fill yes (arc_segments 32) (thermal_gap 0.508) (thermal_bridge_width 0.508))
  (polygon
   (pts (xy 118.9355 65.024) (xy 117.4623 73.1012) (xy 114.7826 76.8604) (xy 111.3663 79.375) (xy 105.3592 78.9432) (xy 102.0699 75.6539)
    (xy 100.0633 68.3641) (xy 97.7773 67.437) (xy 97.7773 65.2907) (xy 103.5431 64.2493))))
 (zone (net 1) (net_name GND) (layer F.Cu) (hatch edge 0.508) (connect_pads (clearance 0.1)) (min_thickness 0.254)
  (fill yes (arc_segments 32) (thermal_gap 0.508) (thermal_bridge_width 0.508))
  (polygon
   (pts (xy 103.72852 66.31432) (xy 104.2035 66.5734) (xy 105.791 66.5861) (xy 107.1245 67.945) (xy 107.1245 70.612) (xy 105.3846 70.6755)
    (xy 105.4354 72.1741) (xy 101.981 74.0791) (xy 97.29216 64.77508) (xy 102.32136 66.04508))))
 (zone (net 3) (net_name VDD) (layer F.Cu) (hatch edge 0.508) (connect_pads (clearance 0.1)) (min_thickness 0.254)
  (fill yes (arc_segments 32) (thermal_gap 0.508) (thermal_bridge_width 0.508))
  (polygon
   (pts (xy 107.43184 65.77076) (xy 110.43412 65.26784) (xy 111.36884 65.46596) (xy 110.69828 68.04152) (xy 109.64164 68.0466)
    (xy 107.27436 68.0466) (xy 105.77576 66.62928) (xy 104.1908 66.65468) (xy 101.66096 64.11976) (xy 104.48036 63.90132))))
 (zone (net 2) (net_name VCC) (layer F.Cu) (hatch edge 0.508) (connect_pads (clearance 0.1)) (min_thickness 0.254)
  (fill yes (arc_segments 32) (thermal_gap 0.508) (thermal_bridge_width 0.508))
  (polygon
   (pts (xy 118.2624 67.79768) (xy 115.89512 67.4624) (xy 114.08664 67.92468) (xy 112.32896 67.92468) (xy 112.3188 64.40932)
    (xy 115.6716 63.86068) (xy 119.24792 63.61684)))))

